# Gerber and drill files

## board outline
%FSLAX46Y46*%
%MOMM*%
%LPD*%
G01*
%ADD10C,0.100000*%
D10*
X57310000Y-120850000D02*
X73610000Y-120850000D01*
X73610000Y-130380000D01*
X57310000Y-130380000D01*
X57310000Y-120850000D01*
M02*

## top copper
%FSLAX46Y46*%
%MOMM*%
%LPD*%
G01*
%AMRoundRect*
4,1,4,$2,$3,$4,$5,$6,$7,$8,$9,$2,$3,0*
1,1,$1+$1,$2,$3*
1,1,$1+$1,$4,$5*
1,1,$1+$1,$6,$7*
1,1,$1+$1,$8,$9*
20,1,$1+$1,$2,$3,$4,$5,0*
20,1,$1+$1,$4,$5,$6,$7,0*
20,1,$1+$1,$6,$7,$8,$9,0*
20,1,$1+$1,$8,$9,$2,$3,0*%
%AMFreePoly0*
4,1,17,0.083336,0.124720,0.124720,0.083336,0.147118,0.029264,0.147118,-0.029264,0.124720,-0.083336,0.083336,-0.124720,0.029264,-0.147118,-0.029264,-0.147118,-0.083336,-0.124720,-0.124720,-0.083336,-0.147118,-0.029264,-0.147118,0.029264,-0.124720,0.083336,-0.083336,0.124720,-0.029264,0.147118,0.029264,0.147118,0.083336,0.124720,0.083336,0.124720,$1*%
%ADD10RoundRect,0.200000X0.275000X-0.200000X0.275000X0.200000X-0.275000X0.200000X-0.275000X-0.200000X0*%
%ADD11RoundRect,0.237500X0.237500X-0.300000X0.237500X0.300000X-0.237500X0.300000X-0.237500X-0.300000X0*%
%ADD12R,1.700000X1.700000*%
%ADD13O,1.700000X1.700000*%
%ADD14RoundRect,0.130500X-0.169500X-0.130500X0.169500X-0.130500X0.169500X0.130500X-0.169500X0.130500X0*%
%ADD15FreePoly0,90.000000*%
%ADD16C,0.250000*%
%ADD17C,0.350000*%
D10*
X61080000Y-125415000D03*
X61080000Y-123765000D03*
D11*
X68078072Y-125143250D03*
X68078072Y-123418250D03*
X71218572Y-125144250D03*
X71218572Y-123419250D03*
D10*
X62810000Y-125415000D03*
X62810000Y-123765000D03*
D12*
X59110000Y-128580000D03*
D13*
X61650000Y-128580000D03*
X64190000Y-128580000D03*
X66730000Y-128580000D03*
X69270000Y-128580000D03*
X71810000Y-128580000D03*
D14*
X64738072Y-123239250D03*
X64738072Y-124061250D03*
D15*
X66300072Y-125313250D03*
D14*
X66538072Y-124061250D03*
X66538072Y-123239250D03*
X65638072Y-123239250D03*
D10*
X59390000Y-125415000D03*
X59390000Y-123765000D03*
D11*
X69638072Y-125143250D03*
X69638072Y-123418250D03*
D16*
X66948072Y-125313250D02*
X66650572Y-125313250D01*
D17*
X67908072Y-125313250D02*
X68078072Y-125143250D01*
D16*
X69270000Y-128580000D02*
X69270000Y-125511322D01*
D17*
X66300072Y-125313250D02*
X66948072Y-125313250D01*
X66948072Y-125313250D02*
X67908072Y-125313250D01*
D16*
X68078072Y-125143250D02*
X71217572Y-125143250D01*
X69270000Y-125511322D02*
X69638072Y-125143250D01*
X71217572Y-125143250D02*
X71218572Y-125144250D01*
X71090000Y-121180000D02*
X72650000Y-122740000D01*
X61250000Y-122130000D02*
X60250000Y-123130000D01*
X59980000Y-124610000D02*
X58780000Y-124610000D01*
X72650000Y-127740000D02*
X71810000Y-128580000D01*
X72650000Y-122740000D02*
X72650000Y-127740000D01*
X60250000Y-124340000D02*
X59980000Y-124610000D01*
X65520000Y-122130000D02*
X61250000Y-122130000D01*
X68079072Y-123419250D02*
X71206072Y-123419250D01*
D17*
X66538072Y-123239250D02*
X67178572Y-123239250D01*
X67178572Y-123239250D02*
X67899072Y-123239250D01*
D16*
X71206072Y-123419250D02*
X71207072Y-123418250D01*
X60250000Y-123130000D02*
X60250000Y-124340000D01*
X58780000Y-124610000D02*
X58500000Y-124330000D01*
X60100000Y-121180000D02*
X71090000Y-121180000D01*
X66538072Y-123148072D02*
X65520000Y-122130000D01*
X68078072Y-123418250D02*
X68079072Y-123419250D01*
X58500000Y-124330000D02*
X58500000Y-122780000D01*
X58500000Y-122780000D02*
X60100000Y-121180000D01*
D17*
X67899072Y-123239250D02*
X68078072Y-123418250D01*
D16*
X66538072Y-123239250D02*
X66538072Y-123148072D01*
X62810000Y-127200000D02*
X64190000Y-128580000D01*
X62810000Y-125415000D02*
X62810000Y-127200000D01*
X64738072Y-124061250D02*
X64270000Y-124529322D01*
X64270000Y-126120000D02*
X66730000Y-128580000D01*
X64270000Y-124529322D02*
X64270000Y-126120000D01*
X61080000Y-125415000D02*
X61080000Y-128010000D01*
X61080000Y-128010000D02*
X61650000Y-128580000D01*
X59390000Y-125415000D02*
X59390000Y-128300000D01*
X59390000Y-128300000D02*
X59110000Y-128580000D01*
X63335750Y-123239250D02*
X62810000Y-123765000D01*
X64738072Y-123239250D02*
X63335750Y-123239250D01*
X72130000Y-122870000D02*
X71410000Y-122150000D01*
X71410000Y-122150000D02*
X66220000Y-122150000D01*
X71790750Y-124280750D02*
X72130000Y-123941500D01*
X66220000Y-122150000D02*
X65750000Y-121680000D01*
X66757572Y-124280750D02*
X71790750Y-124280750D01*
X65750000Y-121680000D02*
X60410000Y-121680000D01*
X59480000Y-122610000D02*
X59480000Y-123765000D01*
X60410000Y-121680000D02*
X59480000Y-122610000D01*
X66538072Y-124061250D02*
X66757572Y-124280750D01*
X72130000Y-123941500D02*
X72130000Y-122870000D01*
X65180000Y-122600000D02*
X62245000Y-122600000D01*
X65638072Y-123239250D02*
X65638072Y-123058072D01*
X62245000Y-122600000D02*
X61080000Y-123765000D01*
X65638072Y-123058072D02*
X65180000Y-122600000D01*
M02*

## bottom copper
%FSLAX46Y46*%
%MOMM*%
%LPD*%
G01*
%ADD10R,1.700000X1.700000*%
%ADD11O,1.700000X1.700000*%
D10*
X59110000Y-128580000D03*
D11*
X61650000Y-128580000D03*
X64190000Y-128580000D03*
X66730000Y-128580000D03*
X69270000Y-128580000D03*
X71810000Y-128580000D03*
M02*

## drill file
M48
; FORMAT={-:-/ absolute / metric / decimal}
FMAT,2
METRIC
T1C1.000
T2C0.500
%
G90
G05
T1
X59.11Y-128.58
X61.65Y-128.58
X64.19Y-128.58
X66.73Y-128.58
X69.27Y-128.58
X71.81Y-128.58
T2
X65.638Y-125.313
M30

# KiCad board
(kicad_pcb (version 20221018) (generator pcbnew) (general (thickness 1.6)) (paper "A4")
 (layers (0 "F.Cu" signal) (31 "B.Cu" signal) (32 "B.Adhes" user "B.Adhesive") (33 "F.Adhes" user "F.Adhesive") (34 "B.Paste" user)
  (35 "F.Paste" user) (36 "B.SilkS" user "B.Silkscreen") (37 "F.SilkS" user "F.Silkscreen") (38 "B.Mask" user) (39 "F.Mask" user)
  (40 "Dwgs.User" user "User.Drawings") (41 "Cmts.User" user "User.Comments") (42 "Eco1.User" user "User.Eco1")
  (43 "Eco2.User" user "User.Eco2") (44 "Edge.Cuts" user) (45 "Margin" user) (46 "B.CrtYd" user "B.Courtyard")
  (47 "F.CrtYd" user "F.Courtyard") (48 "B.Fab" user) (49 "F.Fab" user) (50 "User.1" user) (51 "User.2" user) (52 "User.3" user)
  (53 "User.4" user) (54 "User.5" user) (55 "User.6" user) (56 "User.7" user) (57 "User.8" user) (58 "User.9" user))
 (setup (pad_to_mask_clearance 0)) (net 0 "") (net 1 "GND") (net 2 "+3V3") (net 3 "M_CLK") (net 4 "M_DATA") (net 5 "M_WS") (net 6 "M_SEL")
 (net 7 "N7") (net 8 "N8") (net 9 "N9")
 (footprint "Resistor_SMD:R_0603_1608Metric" (layer "F.Cu") (at 61.08 124.59 90)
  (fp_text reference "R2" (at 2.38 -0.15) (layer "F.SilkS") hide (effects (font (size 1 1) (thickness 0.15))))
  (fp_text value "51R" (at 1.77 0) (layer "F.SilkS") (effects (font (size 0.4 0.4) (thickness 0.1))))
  (pad "1" smd roundrect (at -0.825 0 90) (size 0.8 0.95) (layers "F.Cu" "F.Paste" "F.Mask") (roundrect_rratio 0.25))
  (pad "2" smd roundrect (at 0.825 0 90) (size 0.8 0.95) (layers "F.Cu" "F.Paste" "F.Mask") (roundrect_rratio 0.25)))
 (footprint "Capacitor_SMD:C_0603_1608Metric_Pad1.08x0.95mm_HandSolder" (layer "F.Cu") (at 68.078072 124.28075 90)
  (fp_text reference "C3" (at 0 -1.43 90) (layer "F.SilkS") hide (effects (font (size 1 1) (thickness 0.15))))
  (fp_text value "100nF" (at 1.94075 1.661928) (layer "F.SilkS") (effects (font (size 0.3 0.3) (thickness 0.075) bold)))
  (pad "1" smd roundrect (at -0.8625 0 90) (size 1.075 0.95) (layers "F.Cu" "F.Paste" "F.Mask") (roundrect_rratio 0.25) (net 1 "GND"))
  (pad "2" smd roundrect (at 0.8625 0 90) (size 1.075 0.95) (layers "F.Cu" "F.Paste" "F.Mask") (roundrect_rratio 0.25) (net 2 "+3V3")))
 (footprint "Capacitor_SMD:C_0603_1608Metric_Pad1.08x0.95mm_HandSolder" (layer "F.Cu") (at 71.218572 124.28175 90)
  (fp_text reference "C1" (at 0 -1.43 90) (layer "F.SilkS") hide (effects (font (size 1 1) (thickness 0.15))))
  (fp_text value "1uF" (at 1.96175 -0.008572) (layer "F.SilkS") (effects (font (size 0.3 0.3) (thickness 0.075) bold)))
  (pad "1" smd roundrect (at -0.8625 0 90) (size 1.075 0.95) (layers "F.Cu" "F.Paste" "F.Mask") (roundrect_rratio 0.25) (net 1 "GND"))
  (pad "2" smd roundrect (at 0.8625 0 90) (size 1.075 0.95) (layers "F.Cu" "F.Paste" "F.Mask") (roundrect_rratio 0.25) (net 2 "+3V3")))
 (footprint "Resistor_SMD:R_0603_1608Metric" (layer "F.Cu") (at 62.81 124.59 90)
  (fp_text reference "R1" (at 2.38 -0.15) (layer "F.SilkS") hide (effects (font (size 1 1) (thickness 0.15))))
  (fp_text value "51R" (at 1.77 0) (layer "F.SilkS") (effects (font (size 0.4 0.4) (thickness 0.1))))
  (pad "1" smd roundrect (at -0.825 0 90) (size 0.8 0.95) (layers "F.Cu" "F.Paste" "F.Mask") (roundrect_rratio 0.25))
  (pad "2" smd roundrect (at 0.825 0 90) (size 0.8 0.95) (layers "F.Cu" "F.Paste" "F.Mask") (roundrect_rratio 0.25)))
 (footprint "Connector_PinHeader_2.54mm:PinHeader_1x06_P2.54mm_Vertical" (layer "F.Cu") (at 59.11 128.58 90)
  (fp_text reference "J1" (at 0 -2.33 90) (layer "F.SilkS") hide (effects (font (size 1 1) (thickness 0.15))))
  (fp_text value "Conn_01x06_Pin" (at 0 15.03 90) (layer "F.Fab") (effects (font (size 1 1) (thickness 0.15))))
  (pad "1" thru_hole rect (at 0 0 90) (size 1.7 1.7) (drill 1) (layers "*.Cu" "*.Mask") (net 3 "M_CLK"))
  (pad "2" thru_hole oval (at 0 2.54 90) (size 1.7 1.7) (drill 1) (layers "*.Cu" "*.Mask") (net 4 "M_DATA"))
  (pad "3" thru_hole oval (at 0 5.08 90) (size 1.7 1.7) (drill 1) (layers "*.Cu" "*.Mask") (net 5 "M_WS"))
  (pad "4" thru_hole oval (at 0 7.62 90) (size 1.7 1.7) (drill 1) (layers "*.Cu" "*.Mask") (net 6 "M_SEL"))
  (pad "5" thru_hole oval (at 0 10.16 90) (size 1.7 1.7) (drill 1) (layers "*.Cu" "*.Mask") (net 1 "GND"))
  (pad "6" thru_hole oval (at 0 12.7 90) (size 1.7 1.7) (drill 1) (layers "*.Cu" "*.Mask") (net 2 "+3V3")))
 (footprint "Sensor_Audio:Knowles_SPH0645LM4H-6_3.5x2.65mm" (layer "F.Cu") (at 65.638072 124.60325)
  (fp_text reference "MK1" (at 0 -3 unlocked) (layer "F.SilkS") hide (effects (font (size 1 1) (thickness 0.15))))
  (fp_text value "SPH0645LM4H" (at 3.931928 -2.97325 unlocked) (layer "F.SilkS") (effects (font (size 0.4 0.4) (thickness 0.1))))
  (pad "" np_thru_hole circle (at 0 0.71) (size 0.5 0.5) (drill 0.5) (layers "*.Mask"))
  (pad "1" smd roundrect (at -0.9 -1.364) (size 0.6 0.522) (layers "F.Cu" "F.Paste" "F.Mask") (roundrect_rratio 0.25) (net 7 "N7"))
  (pad "2" smd roundrect (at -0.9 -0.542) (size 0.6 0.522) (layers "F.Cu" "F.Paste" "F.Mask") (roundrect_rratio 0.25) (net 6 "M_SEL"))
  (pad "3" smd custom (at 0.662 0.71 90) (size 0.3 0.3) (layers "F.Cu" "F.Mask") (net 1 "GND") (options (clearance outline) (anchor circle))
   (primitives))
  (pad "4" smd roundrect (at 0.9 -0.542) (size 0.6 0.522) (layers "F.Cu" "F.Paste" "F.Mask") (roundrect_rratio 0.25) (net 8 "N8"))
  (pad "5" smd roundrect (at 0.9 -1.364) (size 0.6 0.522) (layers "F.Cu" "F.Paste" "F.Mask") (roundrect_rratio 0.25) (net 2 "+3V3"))
  (pad "6" smd roundrect (at 0 -1.364) (size 0.6 0.522) (layers "F.Cu" "F.Paste" "F.Mask") (roundrect_rratio 0.25) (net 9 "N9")))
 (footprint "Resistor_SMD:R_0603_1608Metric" (layer "F.Cu") (at 59.39 124.59 90)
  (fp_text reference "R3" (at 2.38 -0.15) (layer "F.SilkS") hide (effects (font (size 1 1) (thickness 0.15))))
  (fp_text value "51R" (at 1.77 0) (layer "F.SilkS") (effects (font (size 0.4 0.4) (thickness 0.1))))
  (pad "1" smd roundrect (at -0.825 0 90) (size 0.8 0.95) (layers "F.Cu" "F.Paste" "F.Mask") (roundrect_rratio 0.25))
  (pad "2" smd roundrect (at 0.825 0 90) (size 0.8 0.95) (layers "F.Cu" "F.Paste" "F.Mask") (roundrect_rratio 0.25)))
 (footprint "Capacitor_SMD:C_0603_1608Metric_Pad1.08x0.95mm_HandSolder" (layer "F.Cu") (at 69.638072 124.28075 90)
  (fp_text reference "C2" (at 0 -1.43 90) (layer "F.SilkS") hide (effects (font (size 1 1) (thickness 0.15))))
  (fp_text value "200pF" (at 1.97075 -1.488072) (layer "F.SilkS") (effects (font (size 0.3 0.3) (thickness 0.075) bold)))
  (pad "1" smd roundrect (at -0.8625 0 90) (size 1.075 0.95) (layers "F.Cu" "F.Paste" "F.Mask") (roundrect_rratio 0.25) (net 1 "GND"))
  (pad "2" smd roundrect (at 0.8625 0 90) (size 1.075 0.95) (layers "F.Cu" "F.Paste" "F.Mask") (roundrect_rratio 0.25) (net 2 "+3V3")))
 (gr_rect (start 57.31 120.85) (end 73.61 130.38) (stroke (width 0.1) (type default)) (fill none) (layer "Edge.Cuts"))
 (segment (start 66.948072 125.31325) (end 66.650572 125.31325) (width 0.25) (layer "F.Cu") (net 1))
 (segment (start 67.908072 125.31325) (end 68.078072 125.14325) (width 0.35) (layer "F.Cu") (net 1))
 (segment (start 69.27 128.58) (end 69.27 125.511322) (width 0.25) (layer "F.Cu") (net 1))
 (segment (start 66.300072 125.31325) (end 66.948072 125.31325) (width 0.35) (layer "F.Cu") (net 1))
 (segment (start 66.948072 125.31325) (end 67.908072 125.31325) (width 0.35) (layer "F.Cu") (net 1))
 (segment (start 68.078072 125.14325) (end 71.217572 125.14325) (width 0.25) (layer "F.Cu") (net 1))
 (segment (start 69.27 125.511322) (end 69.638072 125.14325) (width 0.25) (layer "F.Cu") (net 1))
 (segment (start 71.217572 125.14325) (end 71.218572 125.14425) (width 0.25) (layer "F.Cu") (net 1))
 (segment (start 71.09 121.18) (end 72.65 122.74) (width 0.25) (layer "F.Cu") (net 2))
 (segment (start 61.25 122.13) (end 60.25 123.13) (width 0.25) (layer "F.Cu") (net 2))
 (segment (start 59.98 124.61) (end 58.78 124.61) (width 0.25) (layer "F.Cu") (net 2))
 (segment (start 72.65 127.74) (end 71.81 128.58) (width 0.25) (layer "F.Cu") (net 2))
 (segment (start 72.65 122.74) (end 72.65 127.74) (width 0.25) (layer "F.Cu") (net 2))
 (segment (start 60.25 124.34) (end 59.98 124.61) (width 0.25) (layer "F.Cu") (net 2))
 (segment (start 65.52 122.13) (end 61.25 122.13) (width 0.25) (layer "F.Cu") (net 2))
 (segment (start 68.079072 123.41925) (end 71.206072 123.41925) (width 0.25) (layer "F.Cu") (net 2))
 (segment (start 66.538072 123.23925) (end 67.178572 123.23925) (width 0.35) (layer "F.Cu") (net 2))
 (segment (start 67.178572 123.23925) (end 67.899072 123.23925) (width 0.35) (layer "F.Cu") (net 2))
 (segment (start 71.206072 123.41925) (end 71.207072 123.41825) (width 0.25) (layer "F.Cu") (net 2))
 (segment (start 60.25 123.13) (end 60.25 124.34) (width 0.25) (layer "F.Cu") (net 2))
 (segment (start 58.78 124.61) (end 58.5 124.33) (width 0.25) (layer "F.Cu") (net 2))
 (segment (start 60.1 121.18) (end 71.09 121.18) (width 0.25) (layer "F.Cu") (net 2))
 (segment (start 66.538072 123.148072) (end 65.52 122.13) (width 0.25) (layer "F.Cu") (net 2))
 (segment (start 68.078072 123.41825) (end 68.079072 123.41925) (width 0.25) (layer "F.Cu") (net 2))
 (segment (start 58.5 124.33) (end 58.5 122.78) (width 0.25) (layer "F.Cu") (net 2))
 (segment (start 58.5 122.78) (end 60.1 121.18) (width 0.25) (layer "F.Cu") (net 2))
 (segment (start 67.899072 123.23925) (end 68.078072 123.41825) (width 0.35) (layer "F.Cu") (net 2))
 (segment (start 66.538072 123.23925) (end 66.538072 123.148072) (width 0.25) (layer "F.Cu") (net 2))
 (segment (start 62.81 127.2) (end 64.19 128.58) (width 0.25) (layer "F.Cu") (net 5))
 (segment (start 62.81 125.415) (end 62.81 127.2) (width 0.25) (layer "F.Cu") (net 5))
 (segment (start 64.738072 124.06125) (end 64.27 124.529322) (width 0.25) (layer "F.Cu") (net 6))
 (segment (start 64.27 126.12) (end 66.73 128.58) (width 0.25) (layer "F.Cu") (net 6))
 (segment (start 64.27 124.529322) (end 64.27 126.12) (width 0.25) (layer "F.Cu") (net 6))
 (segment (start 61.08 125.415) (end 61.08 128.01) (width 0.25) (layer "F.Cu") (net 4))
 (segment (start 61.08 128.01) (end 61.65 128.58) (width 0.25) (layer "F.Cu") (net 4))
 (segment (start 59.39 125.415) (end 59.39 128.3) (width 0.25) (layer "F.Cu") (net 3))
 (segment (start 59.39 128.3) (end 59.11 128.58) (width 0.25) (layer "F.Cu") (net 3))
 (segment (start 63.33575 123.23925) (end 62.81 123.765) (width 0.25) (layer "F.Cu") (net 7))
 (segment (start 64.738072 123.23925) (end 63.33575 123.23925) (width 0.25) (layer "F.Cu") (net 7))
 (segment (start 72.13 122.87) (end 71.41 122.15) (width 0.25) (layer "F.Cu") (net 8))
 (segment (start 71.41 122.15) (end 66.22 122.15) (width 0.25) (layer "F.Cu") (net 8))
 (segment (start 71.79075 124.28075) (end 72.13 123.9415) (width 0.25) (layer "F.Cu") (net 8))
 (segment (start 66.22 122.15) (end 65.75 121.68) (width 0.25) (layer "F.Cu") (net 8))
 (segment (start 66.757572 124.28075) (end 71.79075 124.28075) (width 0.25) (layer "F.Cu") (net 8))
 (segment (start 65.75 121.68) (end 60.41 121.68) (width 0.25) (layer "F.Cu") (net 8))
 (segment (start 59.48 122.61) (end 59.48 123.765) (width 0.25) (layer "F.Cu") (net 8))
 (segment (start 60.41 121.68) (end 59.48 122.61) (width 0.25) (layer "F.Cu") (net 8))
 (segment (start 66.538072 124.06125) (end 66.757572 124.28075) (width 0.25) (layer "F.Cu") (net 8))
 (segment (start 72.13 123.9415) (end 72.13 122.87) (width 0.25) (layer "F.Cu") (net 8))
 (segment (start 65.18 122.6) (end 62.245 122.6) (width 0.25) (layer "F.Cu") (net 9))
 (segment (start 65.638072 123.23925) (end 65.638072 123.058072) (width 0.25) (layer "F.Cu") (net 9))
 (segment (start 62.245 122.6) (end 61.08 123.765) (width 0.25) (layer "F.Cu") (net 9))
 (segment (start 65.638072 123.058072) (end 65.18 122.6) (width 0.25) (layer "F.Cu") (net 9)))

